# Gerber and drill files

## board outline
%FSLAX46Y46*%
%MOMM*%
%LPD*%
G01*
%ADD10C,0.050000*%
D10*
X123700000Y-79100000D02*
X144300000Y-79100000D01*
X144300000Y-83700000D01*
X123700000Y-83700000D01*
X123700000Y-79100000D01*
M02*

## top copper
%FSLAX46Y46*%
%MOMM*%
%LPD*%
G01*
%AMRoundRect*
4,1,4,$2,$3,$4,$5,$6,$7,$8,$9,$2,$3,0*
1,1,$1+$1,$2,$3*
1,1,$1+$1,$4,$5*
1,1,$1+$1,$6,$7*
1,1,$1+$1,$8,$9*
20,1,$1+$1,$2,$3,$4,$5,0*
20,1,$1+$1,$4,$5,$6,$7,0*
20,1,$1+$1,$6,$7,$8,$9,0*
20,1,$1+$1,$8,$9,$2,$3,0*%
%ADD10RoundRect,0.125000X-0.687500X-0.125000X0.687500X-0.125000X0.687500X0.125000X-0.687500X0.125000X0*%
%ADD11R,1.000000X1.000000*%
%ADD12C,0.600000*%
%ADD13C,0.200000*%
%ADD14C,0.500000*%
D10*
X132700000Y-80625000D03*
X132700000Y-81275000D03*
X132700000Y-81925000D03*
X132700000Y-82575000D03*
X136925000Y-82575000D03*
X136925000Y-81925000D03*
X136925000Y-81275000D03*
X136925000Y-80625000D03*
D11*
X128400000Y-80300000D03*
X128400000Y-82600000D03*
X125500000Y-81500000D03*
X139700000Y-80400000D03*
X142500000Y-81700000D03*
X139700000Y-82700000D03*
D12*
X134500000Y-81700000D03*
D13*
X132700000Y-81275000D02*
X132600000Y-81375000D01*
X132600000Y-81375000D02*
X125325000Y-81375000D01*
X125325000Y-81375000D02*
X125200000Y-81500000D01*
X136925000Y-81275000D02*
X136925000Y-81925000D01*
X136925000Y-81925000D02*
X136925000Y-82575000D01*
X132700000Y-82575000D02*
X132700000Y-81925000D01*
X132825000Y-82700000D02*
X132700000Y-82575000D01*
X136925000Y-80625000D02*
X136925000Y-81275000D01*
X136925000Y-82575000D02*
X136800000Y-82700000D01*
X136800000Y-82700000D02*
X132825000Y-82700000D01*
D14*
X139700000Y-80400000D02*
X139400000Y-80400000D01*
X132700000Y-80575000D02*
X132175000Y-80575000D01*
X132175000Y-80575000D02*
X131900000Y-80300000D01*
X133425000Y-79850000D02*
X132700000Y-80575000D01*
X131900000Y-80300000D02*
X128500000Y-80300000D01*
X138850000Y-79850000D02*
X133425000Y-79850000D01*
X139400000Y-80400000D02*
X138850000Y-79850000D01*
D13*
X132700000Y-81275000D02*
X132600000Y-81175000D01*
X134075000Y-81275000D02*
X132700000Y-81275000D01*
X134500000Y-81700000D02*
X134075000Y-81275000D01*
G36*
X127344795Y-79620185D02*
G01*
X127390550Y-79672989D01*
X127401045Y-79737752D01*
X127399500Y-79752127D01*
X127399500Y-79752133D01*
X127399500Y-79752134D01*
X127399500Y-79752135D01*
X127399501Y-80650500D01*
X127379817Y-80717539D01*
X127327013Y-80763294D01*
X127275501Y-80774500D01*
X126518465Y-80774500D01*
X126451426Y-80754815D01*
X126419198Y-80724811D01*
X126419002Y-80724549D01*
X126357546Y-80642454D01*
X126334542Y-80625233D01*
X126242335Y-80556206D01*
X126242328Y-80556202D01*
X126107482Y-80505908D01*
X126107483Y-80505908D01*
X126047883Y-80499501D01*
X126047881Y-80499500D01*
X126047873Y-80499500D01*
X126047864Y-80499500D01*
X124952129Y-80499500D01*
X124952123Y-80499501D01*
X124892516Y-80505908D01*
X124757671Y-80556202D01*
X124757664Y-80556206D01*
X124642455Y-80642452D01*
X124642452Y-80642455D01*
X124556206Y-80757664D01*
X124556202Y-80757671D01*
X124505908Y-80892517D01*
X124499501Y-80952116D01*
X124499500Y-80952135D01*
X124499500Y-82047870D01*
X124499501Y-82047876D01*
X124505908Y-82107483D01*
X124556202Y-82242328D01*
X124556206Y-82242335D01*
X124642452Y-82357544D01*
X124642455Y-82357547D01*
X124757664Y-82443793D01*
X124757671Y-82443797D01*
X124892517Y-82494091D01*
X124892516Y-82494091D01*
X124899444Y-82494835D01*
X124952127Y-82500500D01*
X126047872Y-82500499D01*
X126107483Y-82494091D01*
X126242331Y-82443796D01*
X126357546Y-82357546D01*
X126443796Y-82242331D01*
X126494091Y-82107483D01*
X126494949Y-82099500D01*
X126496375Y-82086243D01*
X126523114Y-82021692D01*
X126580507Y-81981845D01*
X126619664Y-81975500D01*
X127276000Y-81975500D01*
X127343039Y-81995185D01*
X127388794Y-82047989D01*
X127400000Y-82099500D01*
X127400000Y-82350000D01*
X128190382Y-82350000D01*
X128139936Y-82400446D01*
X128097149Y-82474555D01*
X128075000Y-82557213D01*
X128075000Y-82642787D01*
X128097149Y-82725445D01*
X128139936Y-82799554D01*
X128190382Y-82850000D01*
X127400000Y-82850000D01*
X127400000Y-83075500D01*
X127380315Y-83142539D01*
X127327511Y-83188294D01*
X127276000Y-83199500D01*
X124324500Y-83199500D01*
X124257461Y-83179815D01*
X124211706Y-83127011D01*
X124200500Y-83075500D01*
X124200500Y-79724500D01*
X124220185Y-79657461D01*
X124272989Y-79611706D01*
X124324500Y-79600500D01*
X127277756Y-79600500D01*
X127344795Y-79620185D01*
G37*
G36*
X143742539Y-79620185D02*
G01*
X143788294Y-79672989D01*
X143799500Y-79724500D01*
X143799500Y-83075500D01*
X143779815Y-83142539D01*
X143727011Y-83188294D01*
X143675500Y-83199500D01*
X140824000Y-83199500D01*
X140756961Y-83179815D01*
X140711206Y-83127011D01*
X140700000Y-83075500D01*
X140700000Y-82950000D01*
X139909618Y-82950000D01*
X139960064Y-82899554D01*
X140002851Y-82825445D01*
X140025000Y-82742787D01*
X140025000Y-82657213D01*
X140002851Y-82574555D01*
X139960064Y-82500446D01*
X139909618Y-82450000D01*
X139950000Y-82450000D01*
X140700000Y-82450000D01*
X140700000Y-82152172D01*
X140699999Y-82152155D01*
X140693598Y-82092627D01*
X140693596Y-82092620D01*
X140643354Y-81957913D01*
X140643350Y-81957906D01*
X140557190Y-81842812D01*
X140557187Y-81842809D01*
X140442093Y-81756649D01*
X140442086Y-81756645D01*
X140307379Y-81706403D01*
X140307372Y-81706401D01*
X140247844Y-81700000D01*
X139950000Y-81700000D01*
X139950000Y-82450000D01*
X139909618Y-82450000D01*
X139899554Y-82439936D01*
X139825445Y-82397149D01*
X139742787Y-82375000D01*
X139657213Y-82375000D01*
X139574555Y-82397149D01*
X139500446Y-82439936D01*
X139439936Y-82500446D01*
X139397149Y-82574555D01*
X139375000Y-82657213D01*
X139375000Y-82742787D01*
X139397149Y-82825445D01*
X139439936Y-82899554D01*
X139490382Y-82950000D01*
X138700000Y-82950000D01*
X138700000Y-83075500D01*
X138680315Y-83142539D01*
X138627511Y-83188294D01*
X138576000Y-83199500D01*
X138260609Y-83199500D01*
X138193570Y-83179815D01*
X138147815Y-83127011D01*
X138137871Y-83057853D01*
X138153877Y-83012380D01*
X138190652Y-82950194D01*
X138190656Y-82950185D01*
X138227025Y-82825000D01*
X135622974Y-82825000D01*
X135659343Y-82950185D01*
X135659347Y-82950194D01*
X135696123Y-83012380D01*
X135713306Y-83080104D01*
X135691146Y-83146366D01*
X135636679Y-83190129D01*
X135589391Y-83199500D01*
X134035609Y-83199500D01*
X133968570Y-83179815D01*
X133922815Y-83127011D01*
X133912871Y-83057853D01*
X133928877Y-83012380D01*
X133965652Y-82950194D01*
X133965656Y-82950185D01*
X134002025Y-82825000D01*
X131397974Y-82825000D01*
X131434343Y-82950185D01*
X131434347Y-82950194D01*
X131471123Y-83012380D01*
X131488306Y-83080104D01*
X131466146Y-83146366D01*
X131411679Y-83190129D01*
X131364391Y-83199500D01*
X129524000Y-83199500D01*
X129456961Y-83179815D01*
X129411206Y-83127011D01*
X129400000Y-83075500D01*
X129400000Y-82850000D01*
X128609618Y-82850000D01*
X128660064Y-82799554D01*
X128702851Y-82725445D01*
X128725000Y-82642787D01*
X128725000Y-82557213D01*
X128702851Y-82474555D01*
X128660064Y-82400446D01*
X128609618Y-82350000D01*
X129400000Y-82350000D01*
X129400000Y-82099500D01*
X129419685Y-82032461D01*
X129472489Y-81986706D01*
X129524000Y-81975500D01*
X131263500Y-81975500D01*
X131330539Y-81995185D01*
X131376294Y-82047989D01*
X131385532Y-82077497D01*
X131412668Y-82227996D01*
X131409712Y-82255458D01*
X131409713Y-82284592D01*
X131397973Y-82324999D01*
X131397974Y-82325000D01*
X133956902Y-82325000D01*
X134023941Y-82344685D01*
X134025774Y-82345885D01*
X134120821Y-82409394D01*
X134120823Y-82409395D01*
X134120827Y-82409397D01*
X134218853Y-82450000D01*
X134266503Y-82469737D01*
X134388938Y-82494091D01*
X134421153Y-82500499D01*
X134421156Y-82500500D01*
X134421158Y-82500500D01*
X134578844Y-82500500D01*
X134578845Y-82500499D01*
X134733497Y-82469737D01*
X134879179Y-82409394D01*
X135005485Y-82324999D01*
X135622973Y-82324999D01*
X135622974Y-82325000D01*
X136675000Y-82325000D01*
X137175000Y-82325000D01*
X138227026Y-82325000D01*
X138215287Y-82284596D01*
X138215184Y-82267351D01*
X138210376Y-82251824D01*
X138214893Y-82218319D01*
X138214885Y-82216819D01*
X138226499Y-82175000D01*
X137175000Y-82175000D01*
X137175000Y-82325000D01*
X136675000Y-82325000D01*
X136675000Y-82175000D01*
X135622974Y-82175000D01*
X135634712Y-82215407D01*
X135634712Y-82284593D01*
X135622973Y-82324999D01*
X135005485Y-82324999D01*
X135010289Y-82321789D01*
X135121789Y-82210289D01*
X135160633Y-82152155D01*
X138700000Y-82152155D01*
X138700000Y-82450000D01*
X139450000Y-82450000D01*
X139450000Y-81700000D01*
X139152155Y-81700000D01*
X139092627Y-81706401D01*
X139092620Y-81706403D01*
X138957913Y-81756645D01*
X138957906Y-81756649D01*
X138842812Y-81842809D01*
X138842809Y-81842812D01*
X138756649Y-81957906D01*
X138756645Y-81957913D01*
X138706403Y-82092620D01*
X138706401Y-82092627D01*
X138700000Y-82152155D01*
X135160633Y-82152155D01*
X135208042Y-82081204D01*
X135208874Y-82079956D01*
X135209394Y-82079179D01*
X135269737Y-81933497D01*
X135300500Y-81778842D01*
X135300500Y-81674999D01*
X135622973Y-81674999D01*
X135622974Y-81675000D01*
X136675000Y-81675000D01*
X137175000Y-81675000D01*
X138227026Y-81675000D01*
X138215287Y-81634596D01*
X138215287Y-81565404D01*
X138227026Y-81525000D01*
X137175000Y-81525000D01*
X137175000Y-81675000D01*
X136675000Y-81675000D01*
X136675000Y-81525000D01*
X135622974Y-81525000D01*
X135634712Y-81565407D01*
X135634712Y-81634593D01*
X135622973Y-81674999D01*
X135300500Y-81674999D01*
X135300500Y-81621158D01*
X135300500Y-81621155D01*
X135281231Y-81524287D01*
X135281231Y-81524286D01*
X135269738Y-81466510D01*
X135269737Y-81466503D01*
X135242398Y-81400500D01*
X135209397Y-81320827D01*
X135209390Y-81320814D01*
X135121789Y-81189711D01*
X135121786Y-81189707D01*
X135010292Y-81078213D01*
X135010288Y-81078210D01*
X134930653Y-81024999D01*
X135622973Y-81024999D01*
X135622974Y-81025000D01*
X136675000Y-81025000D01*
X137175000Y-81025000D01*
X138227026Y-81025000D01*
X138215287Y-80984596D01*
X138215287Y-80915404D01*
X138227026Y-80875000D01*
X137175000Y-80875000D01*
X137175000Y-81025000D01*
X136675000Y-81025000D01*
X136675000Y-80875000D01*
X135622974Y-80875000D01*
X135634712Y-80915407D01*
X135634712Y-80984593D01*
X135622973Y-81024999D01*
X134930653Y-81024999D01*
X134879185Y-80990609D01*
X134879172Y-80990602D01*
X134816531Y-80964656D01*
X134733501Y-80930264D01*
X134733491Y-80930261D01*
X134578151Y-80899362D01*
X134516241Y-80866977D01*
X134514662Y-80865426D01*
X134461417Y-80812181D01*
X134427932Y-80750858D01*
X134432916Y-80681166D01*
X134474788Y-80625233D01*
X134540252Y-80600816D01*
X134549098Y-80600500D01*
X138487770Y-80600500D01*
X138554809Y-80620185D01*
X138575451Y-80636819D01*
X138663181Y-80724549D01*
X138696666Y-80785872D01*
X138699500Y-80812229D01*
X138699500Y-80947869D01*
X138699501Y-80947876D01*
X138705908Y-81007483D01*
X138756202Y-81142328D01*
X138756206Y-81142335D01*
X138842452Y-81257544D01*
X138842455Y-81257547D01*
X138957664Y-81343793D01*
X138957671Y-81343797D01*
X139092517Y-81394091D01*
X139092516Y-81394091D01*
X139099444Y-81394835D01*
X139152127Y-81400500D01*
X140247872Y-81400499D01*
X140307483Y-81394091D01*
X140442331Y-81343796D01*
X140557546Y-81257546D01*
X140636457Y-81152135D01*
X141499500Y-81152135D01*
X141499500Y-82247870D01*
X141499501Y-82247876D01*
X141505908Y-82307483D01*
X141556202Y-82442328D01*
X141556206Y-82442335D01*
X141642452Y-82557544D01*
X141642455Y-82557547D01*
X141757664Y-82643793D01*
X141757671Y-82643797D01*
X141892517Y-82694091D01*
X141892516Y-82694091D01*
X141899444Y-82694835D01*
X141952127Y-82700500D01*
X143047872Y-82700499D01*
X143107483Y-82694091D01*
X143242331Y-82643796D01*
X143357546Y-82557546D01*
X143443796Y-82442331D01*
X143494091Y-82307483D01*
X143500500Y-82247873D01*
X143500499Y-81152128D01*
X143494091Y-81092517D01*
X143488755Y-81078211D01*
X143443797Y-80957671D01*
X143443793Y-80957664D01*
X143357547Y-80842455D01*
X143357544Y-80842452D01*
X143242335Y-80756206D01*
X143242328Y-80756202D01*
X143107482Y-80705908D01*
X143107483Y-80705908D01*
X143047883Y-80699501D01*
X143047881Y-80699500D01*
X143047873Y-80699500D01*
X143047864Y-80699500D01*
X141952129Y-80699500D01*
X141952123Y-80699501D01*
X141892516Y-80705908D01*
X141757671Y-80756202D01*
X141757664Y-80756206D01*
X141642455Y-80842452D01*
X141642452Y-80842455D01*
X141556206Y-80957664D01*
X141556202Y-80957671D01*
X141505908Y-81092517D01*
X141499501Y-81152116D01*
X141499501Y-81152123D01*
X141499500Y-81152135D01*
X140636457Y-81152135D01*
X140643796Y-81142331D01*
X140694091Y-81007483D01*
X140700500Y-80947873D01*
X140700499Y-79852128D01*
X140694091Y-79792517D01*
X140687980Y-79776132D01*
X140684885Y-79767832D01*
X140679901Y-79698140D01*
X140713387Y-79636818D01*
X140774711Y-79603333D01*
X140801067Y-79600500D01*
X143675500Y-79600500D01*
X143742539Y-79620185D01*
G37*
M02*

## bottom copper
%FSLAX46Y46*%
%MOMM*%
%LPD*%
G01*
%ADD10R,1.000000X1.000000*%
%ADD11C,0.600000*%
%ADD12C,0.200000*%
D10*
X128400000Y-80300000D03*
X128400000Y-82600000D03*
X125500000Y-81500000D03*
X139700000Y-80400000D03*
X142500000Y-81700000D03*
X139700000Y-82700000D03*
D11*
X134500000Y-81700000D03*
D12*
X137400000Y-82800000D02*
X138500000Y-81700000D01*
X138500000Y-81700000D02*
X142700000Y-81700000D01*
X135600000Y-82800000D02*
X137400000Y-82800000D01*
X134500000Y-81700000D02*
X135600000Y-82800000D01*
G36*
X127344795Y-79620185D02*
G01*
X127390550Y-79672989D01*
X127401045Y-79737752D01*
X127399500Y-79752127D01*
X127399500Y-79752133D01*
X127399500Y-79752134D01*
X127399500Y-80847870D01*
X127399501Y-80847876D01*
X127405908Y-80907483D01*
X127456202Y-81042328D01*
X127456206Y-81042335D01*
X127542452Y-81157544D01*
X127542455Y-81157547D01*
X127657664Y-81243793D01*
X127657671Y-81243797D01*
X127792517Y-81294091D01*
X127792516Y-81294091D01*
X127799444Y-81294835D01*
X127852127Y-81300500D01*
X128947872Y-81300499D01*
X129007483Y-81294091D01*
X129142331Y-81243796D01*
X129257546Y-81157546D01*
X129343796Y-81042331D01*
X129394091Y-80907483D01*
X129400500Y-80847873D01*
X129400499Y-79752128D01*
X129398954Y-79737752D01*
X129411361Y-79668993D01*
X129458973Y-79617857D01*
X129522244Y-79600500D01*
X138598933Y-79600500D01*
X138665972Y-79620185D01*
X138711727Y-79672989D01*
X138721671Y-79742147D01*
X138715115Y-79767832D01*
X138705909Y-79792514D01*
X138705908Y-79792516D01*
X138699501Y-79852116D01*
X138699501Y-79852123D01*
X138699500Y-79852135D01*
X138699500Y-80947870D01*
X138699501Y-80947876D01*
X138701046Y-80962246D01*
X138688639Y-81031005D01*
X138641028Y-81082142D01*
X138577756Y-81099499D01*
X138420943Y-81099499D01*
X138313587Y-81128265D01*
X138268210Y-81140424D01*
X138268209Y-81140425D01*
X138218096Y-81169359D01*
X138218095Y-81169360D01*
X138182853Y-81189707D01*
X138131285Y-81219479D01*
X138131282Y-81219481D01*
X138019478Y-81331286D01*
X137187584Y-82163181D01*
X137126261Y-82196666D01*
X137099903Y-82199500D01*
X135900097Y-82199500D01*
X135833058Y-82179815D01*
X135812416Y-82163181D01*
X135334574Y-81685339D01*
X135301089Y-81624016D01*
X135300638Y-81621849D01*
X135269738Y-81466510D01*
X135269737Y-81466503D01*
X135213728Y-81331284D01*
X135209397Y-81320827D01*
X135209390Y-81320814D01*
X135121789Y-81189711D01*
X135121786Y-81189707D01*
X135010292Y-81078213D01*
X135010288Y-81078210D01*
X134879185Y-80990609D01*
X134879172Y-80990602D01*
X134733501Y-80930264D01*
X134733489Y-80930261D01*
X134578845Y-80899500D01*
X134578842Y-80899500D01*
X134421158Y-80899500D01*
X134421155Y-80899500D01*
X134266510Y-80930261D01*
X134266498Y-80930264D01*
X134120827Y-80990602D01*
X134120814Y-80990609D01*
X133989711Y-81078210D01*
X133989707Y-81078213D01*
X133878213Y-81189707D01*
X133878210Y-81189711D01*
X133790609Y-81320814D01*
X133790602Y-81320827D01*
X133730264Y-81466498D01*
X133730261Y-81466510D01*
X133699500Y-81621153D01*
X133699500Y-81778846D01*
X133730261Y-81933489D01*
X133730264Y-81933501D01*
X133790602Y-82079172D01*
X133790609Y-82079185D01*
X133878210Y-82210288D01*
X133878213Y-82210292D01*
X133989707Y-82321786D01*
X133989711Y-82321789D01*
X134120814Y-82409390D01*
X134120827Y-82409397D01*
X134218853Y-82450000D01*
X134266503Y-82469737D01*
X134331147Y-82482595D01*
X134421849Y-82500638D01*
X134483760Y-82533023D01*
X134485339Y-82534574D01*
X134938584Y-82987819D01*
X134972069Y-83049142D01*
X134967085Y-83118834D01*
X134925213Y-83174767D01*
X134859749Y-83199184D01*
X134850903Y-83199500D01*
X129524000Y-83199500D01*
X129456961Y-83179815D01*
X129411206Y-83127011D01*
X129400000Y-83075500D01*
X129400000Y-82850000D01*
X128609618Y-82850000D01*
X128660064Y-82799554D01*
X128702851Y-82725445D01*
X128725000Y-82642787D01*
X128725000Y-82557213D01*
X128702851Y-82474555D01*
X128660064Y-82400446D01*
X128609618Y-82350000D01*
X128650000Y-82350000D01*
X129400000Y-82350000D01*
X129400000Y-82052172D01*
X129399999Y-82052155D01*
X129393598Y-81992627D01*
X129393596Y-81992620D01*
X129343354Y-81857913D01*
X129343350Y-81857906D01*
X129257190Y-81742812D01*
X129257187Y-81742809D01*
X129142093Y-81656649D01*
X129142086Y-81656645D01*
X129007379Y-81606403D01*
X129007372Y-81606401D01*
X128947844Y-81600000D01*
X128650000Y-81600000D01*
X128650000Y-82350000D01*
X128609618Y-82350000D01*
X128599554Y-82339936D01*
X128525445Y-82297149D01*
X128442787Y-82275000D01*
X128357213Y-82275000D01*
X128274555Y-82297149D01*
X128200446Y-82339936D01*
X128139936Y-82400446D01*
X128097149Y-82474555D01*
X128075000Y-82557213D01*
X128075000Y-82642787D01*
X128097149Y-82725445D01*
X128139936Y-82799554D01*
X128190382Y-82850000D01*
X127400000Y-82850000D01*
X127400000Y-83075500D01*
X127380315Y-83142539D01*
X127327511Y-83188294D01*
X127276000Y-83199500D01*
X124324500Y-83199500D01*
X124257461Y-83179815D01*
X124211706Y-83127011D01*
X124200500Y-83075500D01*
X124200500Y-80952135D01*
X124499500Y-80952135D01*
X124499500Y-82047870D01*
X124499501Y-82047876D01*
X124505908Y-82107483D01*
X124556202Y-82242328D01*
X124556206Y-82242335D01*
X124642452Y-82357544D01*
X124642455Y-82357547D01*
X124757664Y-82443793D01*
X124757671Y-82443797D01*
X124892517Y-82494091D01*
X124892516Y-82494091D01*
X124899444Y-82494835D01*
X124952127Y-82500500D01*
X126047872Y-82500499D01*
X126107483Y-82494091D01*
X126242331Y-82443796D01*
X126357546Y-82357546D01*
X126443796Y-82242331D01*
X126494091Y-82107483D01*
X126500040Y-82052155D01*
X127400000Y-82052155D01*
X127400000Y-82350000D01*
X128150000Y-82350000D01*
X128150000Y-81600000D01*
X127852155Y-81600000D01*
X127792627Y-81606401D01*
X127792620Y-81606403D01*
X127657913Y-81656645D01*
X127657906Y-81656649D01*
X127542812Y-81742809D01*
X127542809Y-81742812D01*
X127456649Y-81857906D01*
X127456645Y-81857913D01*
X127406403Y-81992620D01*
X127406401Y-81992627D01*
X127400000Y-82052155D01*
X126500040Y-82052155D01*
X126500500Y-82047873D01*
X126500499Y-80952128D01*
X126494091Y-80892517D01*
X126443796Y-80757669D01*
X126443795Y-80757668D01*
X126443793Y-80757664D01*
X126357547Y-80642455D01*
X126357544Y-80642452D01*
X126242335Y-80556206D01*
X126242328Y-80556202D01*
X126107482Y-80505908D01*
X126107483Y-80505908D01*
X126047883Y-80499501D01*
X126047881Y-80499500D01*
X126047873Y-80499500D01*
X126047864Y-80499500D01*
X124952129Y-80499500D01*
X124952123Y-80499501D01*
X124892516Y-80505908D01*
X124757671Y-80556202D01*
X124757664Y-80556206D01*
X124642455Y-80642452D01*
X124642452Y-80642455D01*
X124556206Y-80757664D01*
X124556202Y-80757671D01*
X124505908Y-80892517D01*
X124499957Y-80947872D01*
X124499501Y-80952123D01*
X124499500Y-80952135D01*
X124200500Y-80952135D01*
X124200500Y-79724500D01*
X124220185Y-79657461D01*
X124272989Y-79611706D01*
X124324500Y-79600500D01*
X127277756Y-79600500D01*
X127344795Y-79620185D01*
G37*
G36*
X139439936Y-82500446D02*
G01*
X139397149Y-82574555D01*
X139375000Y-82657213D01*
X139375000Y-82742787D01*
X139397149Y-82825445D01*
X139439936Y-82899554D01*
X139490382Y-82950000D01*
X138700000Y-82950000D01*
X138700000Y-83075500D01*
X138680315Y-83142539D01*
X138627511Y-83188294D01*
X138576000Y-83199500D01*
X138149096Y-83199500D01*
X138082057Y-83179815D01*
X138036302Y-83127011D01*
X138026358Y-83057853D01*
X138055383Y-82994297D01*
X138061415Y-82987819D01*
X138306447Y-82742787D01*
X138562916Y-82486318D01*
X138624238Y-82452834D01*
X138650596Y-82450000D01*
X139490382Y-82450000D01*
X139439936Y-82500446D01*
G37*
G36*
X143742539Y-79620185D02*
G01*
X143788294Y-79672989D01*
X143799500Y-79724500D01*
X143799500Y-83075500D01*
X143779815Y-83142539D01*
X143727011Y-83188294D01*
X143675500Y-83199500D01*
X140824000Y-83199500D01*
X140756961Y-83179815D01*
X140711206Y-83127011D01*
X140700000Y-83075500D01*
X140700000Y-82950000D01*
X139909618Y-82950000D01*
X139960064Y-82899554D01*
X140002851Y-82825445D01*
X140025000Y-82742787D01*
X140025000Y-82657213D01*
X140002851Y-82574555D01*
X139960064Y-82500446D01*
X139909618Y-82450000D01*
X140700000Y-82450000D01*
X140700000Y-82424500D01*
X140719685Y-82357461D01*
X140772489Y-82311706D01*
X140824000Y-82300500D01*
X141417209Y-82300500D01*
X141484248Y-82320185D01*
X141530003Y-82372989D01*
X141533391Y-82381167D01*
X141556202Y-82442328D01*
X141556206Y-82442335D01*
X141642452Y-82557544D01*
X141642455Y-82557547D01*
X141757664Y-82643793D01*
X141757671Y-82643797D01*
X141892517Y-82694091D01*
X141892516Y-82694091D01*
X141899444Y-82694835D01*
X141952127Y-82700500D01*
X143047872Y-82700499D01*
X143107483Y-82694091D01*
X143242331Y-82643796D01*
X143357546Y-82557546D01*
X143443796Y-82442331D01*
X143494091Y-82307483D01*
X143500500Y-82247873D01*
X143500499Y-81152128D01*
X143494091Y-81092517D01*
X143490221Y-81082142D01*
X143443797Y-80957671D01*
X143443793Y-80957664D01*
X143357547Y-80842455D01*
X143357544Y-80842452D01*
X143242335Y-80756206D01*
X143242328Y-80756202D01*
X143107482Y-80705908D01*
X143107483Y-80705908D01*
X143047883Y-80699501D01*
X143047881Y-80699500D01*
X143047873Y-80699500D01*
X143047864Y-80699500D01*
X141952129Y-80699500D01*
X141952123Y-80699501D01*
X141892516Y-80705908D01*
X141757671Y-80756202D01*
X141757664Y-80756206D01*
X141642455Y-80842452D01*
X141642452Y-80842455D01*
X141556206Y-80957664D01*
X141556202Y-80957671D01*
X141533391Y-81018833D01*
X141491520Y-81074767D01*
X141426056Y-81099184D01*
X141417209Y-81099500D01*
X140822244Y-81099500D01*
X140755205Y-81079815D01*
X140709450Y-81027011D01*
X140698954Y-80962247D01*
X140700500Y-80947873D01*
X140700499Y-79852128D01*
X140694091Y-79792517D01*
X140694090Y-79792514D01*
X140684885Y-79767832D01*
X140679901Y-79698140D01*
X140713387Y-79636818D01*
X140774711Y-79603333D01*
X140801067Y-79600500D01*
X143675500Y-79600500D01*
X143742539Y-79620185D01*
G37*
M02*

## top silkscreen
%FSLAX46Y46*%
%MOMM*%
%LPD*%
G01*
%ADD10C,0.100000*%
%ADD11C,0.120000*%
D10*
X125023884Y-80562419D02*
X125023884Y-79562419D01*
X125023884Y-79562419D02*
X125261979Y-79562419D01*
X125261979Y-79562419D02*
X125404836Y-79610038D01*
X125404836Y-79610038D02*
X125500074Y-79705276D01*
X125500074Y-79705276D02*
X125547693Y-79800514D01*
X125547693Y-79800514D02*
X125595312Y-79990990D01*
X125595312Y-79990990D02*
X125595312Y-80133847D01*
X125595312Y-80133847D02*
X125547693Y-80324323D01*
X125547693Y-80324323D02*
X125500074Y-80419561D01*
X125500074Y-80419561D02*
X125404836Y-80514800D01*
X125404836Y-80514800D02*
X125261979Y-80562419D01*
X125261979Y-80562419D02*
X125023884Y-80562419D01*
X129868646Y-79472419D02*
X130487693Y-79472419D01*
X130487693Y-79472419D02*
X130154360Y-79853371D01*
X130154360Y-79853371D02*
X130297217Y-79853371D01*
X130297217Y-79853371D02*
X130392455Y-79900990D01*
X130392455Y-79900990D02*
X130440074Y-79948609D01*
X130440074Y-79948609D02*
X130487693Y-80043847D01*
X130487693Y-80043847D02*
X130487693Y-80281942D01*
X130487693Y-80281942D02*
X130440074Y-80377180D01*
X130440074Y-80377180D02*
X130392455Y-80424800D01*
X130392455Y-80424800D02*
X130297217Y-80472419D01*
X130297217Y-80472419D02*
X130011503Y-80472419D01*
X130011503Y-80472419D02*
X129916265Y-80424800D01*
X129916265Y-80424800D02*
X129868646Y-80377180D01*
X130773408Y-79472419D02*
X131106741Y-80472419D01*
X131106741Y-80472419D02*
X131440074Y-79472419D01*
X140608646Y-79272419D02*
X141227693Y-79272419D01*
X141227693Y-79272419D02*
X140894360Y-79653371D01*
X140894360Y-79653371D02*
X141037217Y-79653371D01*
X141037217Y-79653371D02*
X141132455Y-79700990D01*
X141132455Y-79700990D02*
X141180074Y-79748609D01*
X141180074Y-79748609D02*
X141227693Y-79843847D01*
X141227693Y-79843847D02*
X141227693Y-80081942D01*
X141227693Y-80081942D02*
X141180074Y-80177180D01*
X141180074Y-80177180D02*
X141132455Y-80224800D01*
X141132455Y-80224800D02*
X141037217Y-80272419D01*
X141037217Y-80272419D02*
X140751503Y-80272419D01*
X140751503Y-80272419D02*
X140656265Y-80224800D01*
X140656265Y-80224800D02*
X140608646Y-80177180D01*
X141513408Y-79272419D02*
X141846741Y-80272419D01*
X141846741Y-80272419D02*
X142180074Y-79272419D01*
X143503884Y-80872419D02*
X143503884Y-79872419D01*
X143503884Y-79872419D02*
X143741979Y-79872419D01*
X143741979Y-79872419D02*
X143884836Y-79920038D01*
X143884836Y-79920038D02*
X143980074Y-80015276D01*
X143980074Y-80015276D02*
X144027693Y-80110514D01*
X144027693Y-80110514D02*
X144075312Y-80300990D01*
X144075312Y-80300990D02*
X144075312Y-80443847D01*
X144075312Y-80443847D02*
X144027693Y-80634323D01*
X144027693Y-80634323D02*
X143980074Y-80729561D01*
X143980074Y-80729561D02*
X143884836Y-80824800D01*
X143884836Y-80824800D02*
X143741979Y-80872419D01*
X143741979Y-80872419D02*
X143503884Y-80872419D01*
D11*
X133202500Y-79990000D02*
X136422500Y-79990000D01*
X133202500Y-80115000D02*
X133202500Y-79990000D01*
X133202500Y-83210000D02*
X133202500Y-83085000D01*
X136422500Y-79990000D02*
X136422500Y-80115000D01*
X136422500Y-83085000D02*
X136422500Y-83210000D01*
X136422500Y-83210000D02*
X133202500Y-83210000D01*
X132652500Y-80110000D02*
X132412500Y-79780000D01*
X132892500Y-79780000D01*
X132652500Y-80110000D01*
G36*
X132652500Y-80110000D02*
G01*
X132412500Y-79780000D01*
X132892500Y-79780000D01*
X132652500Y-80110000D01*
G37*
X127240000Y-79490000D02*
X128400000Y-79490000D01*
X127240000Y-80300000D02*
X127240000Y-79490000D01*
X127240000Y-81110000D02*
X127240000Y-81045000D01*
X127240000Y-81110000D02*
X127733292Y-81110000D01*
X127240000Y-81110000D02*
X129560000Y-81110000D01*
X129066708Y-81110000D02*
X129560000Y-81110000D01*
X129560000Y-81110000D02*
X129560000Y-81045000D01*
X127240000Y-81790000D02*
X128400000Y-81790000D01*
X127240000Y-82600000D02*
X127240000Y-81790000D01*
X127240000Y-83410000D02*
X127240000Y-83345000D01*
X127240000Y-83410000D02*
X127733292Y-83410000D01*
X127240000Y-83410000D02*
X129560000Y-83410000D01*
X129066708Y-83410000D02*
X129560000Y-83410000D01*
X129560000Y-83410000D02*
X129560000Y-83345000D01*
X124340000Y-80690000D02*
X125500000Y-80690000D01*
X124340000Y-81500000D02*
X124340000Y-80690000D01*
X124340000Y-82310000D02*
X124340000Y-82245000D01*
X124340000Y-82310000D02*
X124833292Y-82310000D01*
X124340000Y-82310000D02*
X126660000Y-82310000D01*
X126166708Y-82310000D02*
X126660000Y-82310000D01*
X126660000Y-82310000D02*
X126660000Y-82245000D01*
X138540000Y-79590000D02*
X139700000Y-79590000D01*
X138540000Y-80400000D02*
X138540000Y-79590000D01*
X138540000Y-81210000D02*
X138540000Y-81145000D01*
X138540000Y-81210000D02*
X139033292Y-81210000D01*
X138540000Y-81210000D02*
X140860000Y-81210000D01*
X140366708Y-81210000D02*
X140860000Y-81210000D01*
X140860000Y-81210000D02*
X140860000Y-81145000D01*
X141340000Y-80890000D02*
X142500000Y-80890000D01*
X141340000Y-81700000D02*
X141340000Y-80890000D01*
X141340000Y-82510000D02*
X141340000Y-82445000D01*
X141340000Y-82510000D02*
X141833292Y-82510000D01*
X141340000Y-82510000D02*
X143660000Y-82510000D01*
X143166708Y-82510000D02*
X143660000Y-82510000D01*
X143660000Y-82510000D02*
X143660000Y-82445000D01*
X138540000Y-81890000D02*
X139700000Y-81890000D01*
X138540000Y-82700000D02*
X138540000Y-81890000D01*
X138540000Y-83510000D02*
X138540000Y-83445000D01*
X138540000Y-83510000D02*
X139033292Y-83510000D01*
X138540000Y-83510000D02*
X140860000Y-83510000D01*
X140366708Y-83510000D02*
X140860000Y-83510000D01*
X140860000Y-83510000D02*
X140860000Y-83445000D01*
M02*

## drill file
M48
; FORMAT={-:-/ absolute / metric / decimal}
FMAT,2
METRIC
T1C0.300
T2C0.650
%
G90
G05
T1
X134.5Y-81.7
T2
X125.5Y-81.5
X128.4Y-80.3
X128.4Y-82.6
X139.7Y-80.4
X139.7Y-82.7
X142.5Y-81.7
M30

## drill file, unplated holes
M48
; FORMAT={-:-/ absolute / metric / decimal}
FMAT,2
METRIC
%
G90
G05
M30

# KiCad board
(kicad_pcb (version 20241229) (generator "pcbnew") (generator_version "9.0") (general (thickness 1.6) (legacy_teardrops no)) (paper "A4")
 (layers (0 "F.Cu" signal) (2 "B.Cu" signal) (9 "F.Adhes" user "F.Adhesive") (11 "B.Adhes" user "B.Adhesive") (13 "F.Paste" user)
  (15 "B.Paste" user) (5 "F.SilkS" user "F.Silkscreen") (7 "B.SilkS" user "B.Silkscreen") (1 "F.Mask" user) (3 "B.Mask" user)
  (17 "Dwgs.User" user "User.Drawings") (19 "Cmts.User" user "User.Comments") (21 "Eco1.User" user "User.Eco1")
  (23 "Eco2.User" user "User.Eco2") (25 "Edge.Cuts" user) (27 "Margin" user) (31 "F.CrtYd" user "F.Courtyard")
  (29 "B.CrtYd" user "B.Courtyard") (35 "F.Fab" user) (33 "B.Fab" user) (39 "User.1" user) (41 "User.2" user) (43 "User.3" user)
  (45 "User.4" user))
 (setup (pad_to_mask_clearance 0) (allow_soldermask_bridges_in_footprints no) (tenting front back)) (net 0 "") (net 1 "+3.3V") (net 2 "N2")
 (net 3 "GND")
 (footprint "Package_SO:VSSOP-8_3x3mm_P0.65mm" (layer "F.Cu") (at 134.8125 81.6)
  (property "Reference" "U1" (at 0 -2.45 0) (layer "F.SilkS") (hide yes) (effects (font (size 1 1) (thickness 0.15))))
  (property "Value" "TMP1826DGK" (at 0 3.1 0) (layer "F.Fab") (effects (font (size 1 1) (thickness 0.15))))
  (fp_line (start -1.61 -1.61) (end 1.61 -1.61) (stroke (width 0.12) (type solid)) (layer "F.SilkS"))
  (fp_line (start -1.61 -1.485) (end -1.61 -1.61) (stroke (width 0.12) (type solid)) (layer "F.SilkS"))
  (fp_line (start -1.61 1.61) (end -1.61 1.485) (stroke (width 0.12) (type solid)) (layer "F.SilkS"))
  (fp_line (start 1.61 -1.61) (end 1.61 -1.485) (stroke (width 0.12) (type solid)) (layer "F.SilkS"))
  (fp_line (start 1.61 1.485) (end 1.61 1.61) (stroke (width 0.12) (type solid)) (layer "F.SilkS"))
  (fp_line (start 1.61 1.61) (end -1.61 1.61) (stroke (width 0.12) (type solid)) (layer "F.SilkS"))
  (fp_poly (pts (xy -2.16 -1.49) (xy -2.4 -1.82) (xy -1.92 -1.82)) (stroke (width 0.12) (type solid)) (fill yes) (layer "F.SilkS"))
  (pad "1" smd roundrect (at -2.1125 -0.975) (size 1.625 0.5) (layers "F.Cu" "F.Mask" "F.Paste") (roundrect_rratio 0.25) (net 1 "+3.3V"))
  (pad "2" smd roundrect (at -2.1125 -0.325) (size 1.625 0.5) (layers "F.Cu" "F.Mask" "F.Paste") (roundrect_rratio 0.25) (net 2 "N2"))
  (pad "3" smd roundrect (at -2.1125 0.325) (size 1.625 0.5) (layers "F.Cu" "F.Mask" "F.Paste") (roundrect_rratio 0.25) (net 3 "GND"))
  (pad "4" smd roundrect (at -2.1125 0.975) (size 1.625 0.5) (layers "F.Cu" "F.Mask" "F.Paste") (roundrect_rratio 0.25) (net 3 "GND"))
  (pad "5" smd roundrect (at 2.1125 0.975) (size 1.625 0.5) (layers "F.Cu" "F.Mask" "F.Paste") (roundrect_rratio 0.25) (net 3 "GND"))
  (pad "6" smd roundrect (at 2.1125 0.325) (size 1.625 0.5) (layers "F.Cu" "F.Mask" "F.Paste") (roundrect_rratio 0.25) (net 3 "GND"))
  (pad "7" smd roundrect (at 2.1125 -0.325) (size 1.625 0.5) (layers "F.Cu" "F.Mask" "F.Paste") (roundrect_rratio 0.25) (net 3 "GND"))
  (pad "8" smd roundrect (at 2.1125 -0.975) (size 1.625 0.5) (layers "F.Cu" "F.Mask" "F.Paste") (roundrect_rratio 0.25) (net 3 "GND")))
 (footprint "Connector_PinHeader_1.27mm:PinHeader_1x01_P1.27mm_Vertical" (layer "F.Cu") (at 128.4 80.3)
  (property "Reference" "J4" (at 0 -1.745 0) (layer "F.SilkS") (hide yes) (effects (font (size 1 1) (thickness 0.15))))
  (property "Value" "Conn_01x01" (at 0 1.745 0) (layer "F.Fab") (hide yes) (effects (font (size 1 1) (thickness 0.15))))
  (fp_line (start -1.16 -0.81) (end 0 -0.81) (stroke (width 0.12) (type solid)) (layer "F.SilkS"))
  (fp_line (start -1.16 0) (end -1.16 -0.81) (stroke (width 0.12) (type solid)) (layer "F.SilkS"))
  (fp_line (start -1.16 0.81) (end -1.16 0.745) (stroke (width 0.12) (type solid)) (layer "F.SilkS"))
  (fp_line (start -1.16 0.81) (end -0.666708 0.81) (stroke (width 0.12) (type solid)) (layer "F.SilkS"))
  (fp_line (start -1.16 0.81) (end 1.16 0.81) (stroke (width 0.12) (type solid)) (layer "F.SilkS"))
  (fp_line (start 0.666708 0.81) (end 1.16 0.81) (stroke (width 0.12) (type solid)) (layer "F.SilkS"))
  (fp_line (start 1.16 0.81) (end 1.16 0.745) (stroke (width 0.12) (type solid)) (layer "F.SilkS"))
  (pad "1" thru_hole rect (at 0 0) (size 1 1) (drill 0.65) (layers "*.Cu" "*.Mask") (remove_unused_layers no) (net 1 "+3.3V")))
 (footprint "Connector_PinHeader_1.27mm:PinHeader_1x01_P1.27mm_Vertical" (layer "F.Cu") (at 128.4 82.6)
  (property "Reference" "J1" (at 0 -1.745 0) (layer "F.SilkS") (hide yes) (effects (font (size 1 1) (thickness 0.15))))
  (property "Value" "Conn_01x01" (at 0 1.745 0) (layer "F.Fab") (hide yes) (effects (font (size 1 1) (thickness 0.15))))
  (fp_line (start -1.16 -0.81) (end 0 -0.81) (stroke (width 0.12) (type solid)) (layer "F.SilkS"))
  (fp_line (start -1.16 0) (end -1.16 -0.81) (stroke (width 0.12) (type solid)) (layer "F.SilkS"))
  (fp_line (start -1.16 0.81) (end -1.16 0.745) (stroke (width 0.12) (type solid)) (layer "F.SilkS"))
  (fp_line (start -1.16 0.81) (end -0.666708 0.81) (stroke (width 0.12) (type solid)) (layer "F.SilkS"))
  (fp_line (start -1.16 0.81) (end 1.16 0.81) (stroke (width 0.12) (type solid)) (layer "F.SilkS"))
  (fp_line (start 0.666708 0.81) (end 1.16 0.81) (stroke (width 0.12) (type solid)) (layer "F.SilkS"))
  (fp_line (start 1.16 0.81) (end 1.16 0.745) (stroke (width 0.12) (type solid)) (layer "F.SilkS"))
  (pad "1" thru_hole rect (at 0 0) (size 1 1) (drill 0.65) (layers "*.Cu" "*.Mask") (remove_unused_layers no) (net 3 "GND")))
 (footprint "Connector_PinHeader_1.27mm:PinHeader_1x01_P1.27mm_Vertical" (layer "F.Cu") (at 125.5 81.5)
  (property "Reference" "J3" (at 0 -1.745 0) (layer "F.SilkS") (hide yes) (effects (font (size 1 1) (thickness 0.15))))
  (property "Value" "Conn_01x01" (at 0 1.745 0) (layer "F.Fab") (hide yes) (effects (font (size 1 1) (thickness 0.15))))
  (fp_line (start -1.16 -0.81) (end 0 -0.81) (stroke (width 0.12) (type solid)) (layer "F.SilkS"))
  (fp_line (start -1.16 0) (end -1.16 -0.81) (stroke (width 0.12) (type solid)) (layer "F.SilkS"))
  (fp_line (start -1.16 0.81) (end -1.16 0.745) (stroke (width 0.12) (type solid)) (layer "F.SilkS"))
  (fp_line (start -1.16 0.81) (end -0.666708 0.81) (stroke (width 0.12) (type solid)) (layer "F.SilkS"))
  (fp_line (start -1.16 0.81) (end 1.16 0.81) (stroke (width 0.12) (type solid)) (layer "F.SilkS"))
  (fp_line (start 0.666708 0.81) (end 1.16 0.81) (stroke (width 0.12) (type solid)) (layer "F.SilkS"))
  (fp_line (start 1.16 0.81) (end 1.16 0.745) (stroke (width 0.12) (type solid)) (layer "F.SilkS"))
  (pad "1" thru_hole rect (at 0 0) (size 1 1) (drill 0.65) (layers "*.Cu" "*.Mask") (remove_unused_layers no) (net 2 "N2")))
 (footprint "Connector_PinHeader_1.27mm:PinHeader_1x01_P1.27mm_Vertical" (layer "F.Cu") (at 139.7 80.4)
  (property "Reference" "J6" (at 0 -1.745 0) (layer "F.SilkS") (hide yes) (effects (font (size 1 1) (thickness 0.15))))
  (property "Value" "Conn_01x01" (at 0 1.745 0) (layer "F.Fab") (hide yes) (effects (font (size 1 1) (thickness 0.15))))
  (fp_line (start -1.16 -0.81) (end 0 -0.81) (stroke (width 0.12) (type solid)) (layer "F.SilkS"))
  (fp_line (start -1.16 0) (end -1.16 -0.81) (stroke (width 0.12) (type solid)) (layer "F.SilkS"))
  (fp_line (start -1.16 0.81) (end -1.16 0.745) (stroke (width 0.12) (type solid)) (layer "F.SilkS"))
  (fp_line (start -1.16 0.81) (end -0.666708 0.81) (stroke (width 0.12) (type solid)) (layer "F.SilkS"))
  (fp_line (start -1.16 0.81) (end 1.16 0.81) (stroke (width 0.12) (type solid)) (layer "F.SilkS"))
  (fp_line (start 0.666708 0.81) (end 1.16 0.81) (stroke (width 0.12) (type solid)) (layer "F.SilkS"))
  (fp_line (start 1.16 0.81) (end 1.16 0.745) (stroke (width 0.12) (type solid)) (layer "F.SilkS"))
  (pad "1" thru_hole rect (at 0 0) (size 1 1) (drill 0.65) (layers "*.Cu" "*.Mask") (remove_unused_layers no) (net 1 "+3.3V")))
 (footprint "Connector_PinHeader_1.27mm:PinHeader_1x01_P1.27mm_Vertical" (layer "F.Cu") (at 142.5 81.7)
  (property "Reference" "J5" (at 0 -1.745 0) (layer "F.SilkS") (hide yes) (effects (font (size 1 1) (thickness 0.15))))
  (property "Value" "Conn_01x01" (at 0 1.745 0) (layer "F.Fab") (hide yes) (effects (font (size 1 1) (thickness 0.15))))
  (fp_line (start -1.16 -0.81) (end 0 -0.81) (stroke (width 0.12) (type solid)) (layer "F.SilkS"))
  (fp_line (start -1.16 0) (end -1.16 -0.81) (stroke (width 0.12) (type solid)) (layer "F.SilkS"))
  (fp_line (start -1.16 0.81) (end -1.16 0.745) (stroke (width 0.12) (type solid)) (layer "F.SilkS"))
  (fp_line (start -1.16 0.81) (end -0.666708 0.81) (stroke (width 0.12) (type solid)) (layer "F.SilkS"))
  (fp_line (start -1.16 0.81) (end 1.16 0.81) (stroke (width 0.12) (type solid)) (layer "F.SilkS"))
  (fp_line (start 0.666708 0.81) (end 1.16 0.81) (stroke (width 0.12) (type solid)) (layer "F.SilkS"))
  (fp_line (start 1.16 0.81) (end 1.16 0.745) (stroke (width 0.12) (type solid)) (layer "F.SilkS"))
  (pad "1" thru_hole rect (at 0 0) (size 1 1) (drill 0.65) (layers "*.Cu" "*.Mask") (remove_unused_layers no) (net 2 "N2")))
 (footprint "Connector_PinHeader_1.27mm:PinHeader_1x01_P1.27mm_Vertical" (layer "F.Cu") (at 139.7 82.7)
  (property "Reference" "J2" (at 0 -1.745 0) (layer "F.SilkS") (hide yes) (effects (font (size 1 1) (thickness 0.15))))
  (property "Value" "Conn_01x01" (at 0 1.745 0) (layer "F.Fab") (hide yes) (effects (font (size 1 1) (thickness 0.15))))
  (fp_line (start -1.16 -0.81) (end 0 -0.81) (stroke (width 0.12) (type solid)) (layer "F.SilkS"))
  (fp_line (start -1.16 0) (end -1.16 -0.81) (stroke (width 0.12) (type solid)) (layer "F.SilkS"))
  (fp_line (start -1.16 0.81) (end -1.16 0.745) (stroke (width 0.12) (type solid)) (layer "F.SilkS"))
  (fp_line (start -1.16 0.81) (end -0.666708 0.81) (stroke (width 0.12) (type solid)) (layer "F.SilkS"))
  (fp_line (start -1.16 0.81) (end 1.16 0.81) (stroke (width 0.12) (type solid)) (layer "F.SilkS"))
  (fp_line (start 0.666708 0.81) (end 1.16 0.81) (stroke (width 0.12) (type solid)) (layer "F.SilkS"))
  (fp_line (start 1.16 0.81) (end 1.16 0.745) (stroke (width 0.12) (type solid)) (layer "F.SilkS"))
  (pad "1" thru_hole rect (at 0 0) (size 1 1) (drill 0.65) (layers "*.Cu" "*.Mask") (remove_unused_layers no) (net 3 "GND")))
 (gr_rect (start 123.7 79.1) (end 144.3 83.7) (stroke (width 0.05) (type default)) (fill no) (layer "Edge.Cuts"))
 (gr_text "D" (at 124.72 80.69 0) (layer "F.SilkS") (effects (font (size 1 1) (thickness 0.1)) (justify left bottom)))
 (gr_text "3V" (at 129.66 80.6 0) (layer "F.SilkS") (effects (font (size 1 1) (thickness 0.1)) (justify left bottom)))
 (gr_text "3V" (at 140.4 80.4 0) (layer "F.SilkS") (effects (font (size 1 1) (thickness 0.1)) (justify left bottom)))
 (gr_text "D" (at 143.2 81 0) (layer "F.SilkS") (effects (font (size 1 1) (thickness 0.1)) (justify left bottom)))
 (segment (start 136.925 81.275) (end 136.925 81.925) (width 0.2) (layer "F.Cu") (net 3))
 (segment (start 136.925 81.925) (end 136.925 82.575) (width 0.2) (layer "F.Cu") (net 3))
 (segment (start 132.7 82.575) (end 132.7 81.925) (width 0.2) (layer "F.Cu") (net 3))
 (segment (start 132.825 82.7) (end 132.7 82.575) (width 0.2) (layer "F.Cu") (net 3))
 (segment (start 136.925 80.625) (end 136.925 81.275) (width 0.2) (layer "F.Cu") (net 3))
 (segment (start 136.925 82.575) (end 136.8 82.7) (width 0.2) (layer "F.Cu") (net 3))
 (segment (start 136.8 82.7) (end 132.825 82.7) (width 0.2) (layer "F.Cu") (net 3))
 (segment (start 139.7 80.4) (end 139.4 80.4) (width 0.5) (layer "F.Cu") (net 1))
 (segment (start 132.7 80.575) (end 132.175 80.575) (width 0.5) (layer "F.Cu") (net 1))
 (segment (start 132.175 80.575) (end 131.9 80.3) (width 0.5) (layer "F.Cu") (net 1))
 (segment (start 133.425 79.85) (end 132.7 80.575) (width 0.5) (layer "F.Cu") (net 1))
 (segment (start 131.9 80.3) (end 128.5 80.3) (width 0.5) (layer "F.Cu") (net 1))
 (segment (start 138.85 79.85) (end 133.425 79.85) (width 0.5) (layer "F.Cu") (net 1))
 (segment (start 139.4 80.4) (end 138.85 79.85) (width 0.5) (layer "F.Cu") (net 1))
 (segment (start 132.7 81.275) (end 132.6 81.175) (width 0.2) (layer "F.Cu") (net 2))
 (segment (start 125.325 81.375) (end 125.2 81.5) (width 0.2) (layer "F.Cu") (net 2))
 (segment (start 134.075 81.275) (end 132.7 81.275) (width 0.2) (layer "F.Cu") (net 2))
 (segment (start 132.7 81.275) (end 132.6 81.375) (width 0.2) (layer "F.Cu") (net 2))
 (segment (start 132.6 81.375) (end 125.325 81.375) (width 0.2) (layer "F.Cu") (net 2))
 (segment (start 134.5 81.7) (end 134.075 81.275) (width 0.2) (layer "F.Cu") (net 2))
 (via (at 134.5 81.7) (size 0.6) (drill 0.3) (layers "F.Cu" "B.Cu") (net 2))
 (segment (start 137.4 82.8) (end 138.5 81.7) (width 0.2) (layer "B.Cu") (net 2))
 (segment (start 138.5 81.7) (end 142.7 81.7) (width 0.2) (layer "B.Cu") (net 2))
 (segment (start 135.6 82.8) (end 137.4 82.8) (width 0.2) (layer "B.Cu") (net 2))
 (segment (start 134.5 81.7) (end 135.6 82.8) (width 0.2) (layer "B.Cu") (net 2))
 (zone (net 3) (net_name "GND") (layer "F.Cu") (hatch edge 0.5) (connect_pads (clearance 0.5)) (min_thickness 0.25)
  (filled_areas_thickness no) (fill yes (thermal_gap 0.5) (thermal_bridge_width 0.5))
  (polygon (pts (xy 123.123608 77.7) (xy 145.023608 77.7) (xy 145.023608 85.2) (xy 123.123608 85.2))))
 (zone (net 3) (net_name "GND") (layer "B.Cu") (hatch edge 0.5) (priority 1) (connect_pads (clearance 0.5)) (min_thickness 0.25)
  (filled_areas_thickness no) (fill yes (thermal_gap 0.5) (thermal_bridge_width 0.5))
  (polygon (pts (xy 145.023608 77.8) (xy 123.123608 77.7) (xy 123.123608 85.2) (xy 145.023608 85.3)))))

